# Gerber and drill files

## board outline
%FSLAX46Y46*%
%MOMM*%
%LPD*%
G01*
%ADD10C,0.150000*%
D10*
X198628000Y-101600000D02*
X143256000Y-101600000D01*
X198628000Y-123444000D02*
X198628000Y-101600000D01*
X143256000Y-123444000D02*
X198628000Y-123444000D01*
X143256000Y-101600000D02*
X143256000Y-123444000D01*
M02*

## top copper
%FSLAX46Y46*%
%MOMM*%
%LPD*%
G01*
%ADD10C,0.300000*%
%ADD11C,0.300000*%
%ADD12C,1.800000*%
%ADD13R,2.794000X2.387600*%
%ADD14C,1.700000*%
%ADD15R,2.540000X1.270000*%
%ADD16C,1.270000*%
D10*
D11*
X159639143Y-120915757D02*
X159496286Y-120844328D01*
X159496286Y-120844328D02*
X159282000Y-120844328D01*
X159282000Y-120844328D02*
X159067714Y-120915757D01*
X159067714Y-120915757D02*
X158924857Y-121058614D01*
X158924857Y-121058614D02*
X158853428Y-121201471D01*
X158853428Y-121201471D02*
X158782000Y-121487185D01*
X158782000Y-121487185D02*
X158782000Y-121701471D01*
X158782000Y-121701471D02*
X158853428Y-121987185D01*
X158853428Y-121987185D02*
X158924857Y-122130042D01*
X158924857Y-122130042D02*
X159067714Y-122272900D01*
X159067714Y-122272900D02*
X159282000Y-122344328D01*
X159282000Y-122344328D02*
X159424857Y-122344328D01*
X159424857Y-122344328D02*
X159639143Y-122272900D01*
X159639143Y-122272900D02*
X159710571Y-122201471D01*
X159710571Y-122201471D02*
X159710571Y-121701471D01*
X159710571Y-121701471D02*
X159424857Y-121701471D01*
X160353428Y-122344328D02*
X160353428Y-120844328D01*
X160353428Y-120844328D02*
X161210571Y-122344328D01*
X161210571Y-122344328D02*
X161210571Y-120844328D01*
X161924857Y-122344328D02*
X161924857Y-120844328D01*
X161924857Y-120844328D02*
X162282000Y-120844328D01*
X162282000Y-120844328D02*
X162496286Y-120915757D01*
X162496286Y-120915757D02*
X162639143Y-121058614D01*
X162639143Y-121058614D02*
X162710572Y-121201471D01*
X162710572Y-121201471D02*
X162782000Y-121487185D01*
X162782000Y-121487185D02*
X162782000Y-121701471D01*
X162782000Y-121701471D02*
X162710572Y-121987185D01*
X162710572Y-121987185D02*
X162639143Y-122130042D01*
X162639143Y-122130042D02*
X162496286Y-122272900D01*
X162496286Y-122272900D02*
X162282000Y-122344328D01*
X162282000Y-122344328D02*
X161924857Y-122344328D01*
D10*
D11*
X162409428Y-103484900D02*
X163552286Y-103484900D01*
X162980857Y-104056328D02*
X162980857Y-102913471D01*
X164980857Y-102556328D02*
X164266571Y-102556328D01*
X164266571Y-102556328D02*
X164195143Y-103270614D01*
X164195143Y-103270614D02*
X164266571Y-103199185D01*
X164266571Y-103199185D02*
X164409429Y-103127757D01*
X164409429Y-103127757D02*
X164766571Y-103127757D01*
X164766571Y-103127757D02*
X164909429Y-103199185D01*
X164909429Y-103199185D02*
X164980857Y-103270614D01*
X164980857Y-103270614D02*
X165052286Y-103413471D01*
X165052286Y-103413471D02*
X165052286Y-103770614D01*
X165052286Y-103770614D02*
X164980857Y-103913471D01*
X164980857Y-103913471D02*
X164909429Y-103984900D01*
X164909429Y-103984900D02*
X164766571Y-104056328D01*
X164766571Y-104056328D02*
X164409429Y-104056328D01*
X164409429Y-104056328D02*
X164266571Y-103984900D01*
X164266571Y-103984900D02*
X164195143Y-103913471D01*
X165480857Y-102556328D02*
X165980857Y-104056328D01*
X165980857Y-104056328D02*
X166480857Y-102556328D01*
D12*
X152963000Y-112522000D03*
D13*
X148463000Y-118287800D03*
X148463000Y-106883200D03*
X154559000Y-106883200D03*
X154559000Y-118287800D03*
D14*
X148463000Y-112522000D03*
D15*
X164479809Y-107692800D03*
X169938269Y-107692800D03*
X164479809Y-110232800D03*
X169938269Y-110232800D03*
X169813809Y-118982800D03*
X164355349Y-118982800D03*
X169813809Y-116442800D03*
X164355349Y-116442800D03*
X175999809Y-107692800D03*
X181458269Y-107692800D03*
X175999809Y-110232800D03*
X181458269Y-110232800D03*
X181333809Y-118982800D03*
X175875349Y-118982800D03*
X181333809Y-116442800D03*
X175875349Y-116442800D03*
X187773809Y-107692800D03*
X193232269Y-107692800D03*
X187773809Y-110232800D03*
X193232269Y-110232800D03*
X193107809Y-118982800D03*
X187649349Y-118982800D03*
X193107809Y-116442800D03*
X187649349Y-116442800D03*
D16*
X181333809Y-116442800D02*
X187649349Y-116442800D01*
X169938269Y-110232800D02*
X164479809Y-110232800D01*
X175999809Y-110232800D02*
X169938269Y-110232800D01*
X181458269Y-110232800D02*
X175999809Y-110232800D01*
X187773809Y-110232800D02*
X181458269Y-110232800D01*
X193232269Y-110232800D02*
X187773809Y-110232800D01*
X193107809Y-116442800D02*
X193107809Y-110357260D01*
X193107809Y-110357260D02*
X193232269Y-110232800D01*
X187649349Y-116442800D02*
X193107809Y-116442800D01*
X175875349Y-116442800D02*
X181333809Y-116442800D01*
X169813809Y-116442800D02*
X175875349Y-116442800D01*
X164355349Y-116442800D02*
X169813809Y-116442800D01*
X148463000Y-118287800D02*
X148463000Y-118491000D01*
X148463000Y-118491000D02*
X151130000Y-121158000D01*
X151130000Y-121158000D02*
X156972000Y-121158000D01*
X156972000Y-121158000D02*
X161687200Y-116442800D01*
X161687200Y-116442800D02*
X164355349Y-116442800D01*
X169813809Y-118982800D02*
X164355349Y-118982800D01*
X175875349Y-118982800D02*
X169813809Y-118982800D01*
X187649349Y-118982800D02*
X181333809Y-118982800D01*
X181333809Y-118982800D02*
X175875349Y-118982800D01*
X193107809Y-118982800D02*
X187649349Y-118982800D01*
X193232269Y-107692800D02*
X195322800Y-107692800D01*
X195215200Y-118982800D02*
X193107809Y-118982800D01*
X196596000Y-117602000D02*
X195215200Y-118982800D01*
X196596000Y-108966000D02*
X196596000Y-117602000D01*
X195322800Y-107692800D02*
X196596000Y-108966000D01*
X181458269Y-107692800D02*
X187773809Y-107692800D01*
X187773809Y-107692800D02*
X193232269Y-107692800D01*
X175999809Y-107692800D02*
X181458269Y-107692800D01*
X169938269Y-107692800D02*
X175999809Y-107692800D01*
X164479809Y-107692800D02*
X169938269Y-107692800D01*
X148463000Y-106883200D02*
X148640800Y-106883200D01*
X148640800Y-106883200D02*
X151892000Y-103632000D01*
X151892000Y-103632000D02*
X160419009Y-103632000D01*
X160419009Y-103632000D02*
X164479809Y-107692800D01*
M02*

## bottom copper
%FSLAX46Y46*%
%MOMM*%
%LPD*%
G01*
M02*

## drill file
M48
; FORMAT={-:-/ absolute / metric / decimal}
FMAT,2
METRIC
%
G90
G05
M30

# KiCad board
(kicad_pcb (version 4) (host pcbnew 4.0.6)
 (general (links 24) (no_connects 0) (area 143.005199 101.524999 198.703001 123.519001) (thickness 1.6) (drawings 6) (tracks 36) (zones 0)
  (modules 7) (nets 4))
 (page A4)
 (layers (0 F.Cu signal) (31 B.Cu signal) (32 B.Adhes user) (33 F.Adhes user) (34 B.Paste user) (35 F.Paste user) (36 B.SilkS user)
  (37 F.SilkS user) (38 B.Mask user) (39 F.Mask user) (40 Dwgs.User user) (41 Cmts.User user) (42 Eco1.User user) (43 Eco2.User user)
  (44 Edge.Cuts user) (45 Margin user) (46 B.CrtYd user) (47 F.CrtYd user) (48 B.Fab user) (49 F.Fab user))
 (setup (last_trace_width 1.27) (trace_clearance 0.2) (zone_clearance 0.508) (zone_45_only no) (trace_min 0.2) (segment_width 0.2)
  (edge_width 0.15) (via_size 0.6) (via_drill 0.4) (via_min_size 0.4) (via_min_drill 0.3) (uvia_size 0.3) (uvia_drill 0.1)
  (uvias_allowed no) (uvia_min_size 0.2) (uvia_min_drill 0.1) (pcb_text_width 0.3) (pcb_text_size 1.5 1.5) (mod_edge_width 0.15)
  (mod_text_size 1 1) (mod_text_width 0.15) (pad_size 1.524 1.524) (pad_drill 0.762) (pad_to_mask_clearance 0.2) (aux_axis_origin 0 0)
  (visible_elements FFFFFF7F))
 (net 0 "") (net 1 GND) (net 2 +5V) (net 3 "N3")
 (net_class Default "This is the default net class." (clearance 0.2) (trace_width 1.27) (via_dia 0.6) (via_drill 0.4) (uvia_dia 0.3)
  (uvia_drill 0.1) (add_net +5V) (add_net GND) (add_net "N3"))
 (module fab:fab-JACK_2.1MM (layer F.Cu) (at 150.876 112.522 270)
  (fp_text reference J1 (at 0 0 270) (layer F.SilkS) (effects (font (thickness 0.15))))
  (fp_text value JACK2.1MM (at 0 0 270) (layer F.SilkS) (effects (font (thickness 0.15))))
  (pad A smd circle (at 0 -2.087 270) (size 1.8 1.8) (layers F.Cu F.Paste F.Mask))
  (pad CONT smd rect (at 5.7658 2.413 270) (size 2.3876 2.794) (layers F.Cu F.Paste F.Mask) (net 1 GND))
  (pad PIN smd rect (at -5.6388 2.413 270) (size 2.3876 2.794) (layers F.Cu F.Paste F.Mask) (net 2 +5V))
  (pad PIN1 smd rect (at -5.6388 -3.683 270) (size 2.3876 2.794) (layers F.Cu F.Paste F.Mask))
  (pad SHUN smd rect (at 5.7658 -3.683 270) (size 2.3876 2.794) (layers F.Cu F.Paste F.Mask) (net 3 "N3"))
  (pad A smd circle (at 0 2.413 270) (size 1.7 1.7) (layers F.Cu F.Paste F.Mask)))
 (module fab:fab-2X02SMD (layer F.Cu) (at 167.019809 108.9628)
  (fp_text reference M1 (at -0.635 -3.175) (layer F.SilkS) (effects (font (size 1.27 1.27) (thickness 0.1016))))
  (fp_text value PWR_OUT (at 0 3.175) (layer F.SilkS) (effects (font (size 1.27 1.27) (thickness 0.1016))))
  (pad 1 smd rect (at -2.54 -1.27) (size 2.54 1.27) (layers F.Cu F.Paste F.Mask) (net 2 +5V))
  (pad 2 smd rect (at 2.91846 -1.27) (size 2.54 1.27) (layers F.Cu F.Paste F.Mask) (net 2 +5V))
  (pad 3 smd rect (at -2.54 1.27) (size 2.54 1.27) (layers F.Cu F.Paste F.Mask) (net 1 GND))
  (pad 4 smd rect (at 2.91846 1.27) (size 2.54 1.27) (layers F.Cu F.Paste F.Mask) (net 1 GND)))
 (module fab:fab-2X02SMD (layer F.Cu) (at 167.273809 117.7128 180)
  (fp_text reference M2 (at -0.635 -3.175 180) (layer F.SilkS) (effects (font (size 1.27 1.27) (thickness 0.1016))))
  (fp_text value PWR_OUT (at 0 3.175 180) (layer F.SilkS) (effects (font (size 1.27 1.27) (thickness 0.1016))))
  (pad 1 smd rect (at -2.54 -1.27 180) (size 2.54 1.27) (layers F.Cu F.Paste F.Mask) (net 2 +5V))
  (pad 2 smd rect (at 2.91846 -1.27 180) (size 2.54 1.27) (layers F.Cu F.Paste F.Mask) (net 2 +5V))
  (pad 3 smd rect (at -2.54 1.27 180) (size 2.54 1.27) (layers F.Cu F.Paste F.Mask) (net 1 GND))
  (pad 4 smd rect (at 2.91846 1.27 180) (size 2.54 1.27) (layers F.Cu F.Paste F.Mask) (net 1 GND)))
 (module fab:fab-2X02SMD (layer F.Cu) (at 178.539809 108.9628)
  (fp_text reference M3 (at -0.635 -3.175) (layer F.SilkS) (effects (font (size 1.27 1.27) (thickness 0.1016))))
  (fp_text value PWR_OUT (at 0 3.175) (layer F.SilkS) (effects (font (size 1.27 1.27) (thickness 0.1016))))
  (pad 1 smd rect (at -2.54 -1.27) (size 2.54 1.27) (layers F.Cu F.Paste F.Mask) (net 2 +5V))
  (pad 2 smd rect (at 2.91846 -1.27) (size 2.54 1.27) (layers F.Cu F.Paste F.Mask) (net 2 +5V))
  (pad 3 smd rect (at -2.54 1.27) (size 2.54 1.27) (layers F.Cu F.Paste F.Mask) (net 1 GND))
  (pad 4 smd rect (at 2.91846 1.27) (size 2.54 1.27) (layers F.Cu F.Paste F.Mask) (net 1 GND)))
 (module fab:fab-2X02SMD (layer F.Cu) (at 178.793809 117.7128 180)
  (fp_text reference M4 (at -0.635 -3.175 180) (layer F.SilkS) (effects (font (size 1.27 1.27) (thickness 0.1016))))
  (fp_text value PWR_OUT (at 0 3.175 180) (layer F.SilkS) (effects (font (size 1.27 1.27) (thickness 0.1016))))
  (pad 1 smd rect (at -2.54 -1.27 180) (size 2.54 1.27) (layers F.Cu F.Paste F.Mask) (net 2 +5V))
  (pad 2 smd rect (at 2.91846 -1.27 180) (size 2.54 1.27) (layers F.Cu F.Paste F.Mask) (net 2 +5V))
  (pad 3 smd rect (at -2.54 1.27 180) (size 2.54 1.27) (layers F.Cu F.Paste F.Mask) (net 1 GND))
  (pad 4 smd rect (at 2.91846 1.27 180) (size 2.54 1.27) (layers F.Cu F.Paste F.Mask) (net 1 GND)))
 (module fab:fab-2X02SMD (layer F.Cu) (at 190.313809 108.9628)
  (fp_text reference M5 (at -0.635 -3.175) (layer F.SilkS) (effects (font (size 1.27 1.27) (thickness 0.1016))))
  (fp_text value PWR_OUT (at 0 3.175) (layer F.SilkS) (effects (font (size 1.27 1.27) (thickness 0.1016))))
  (pad 1 smd rect (at -2.54 -1.27) (size 2.54 1.27) (layers F.Cu F.Paste F.Mask) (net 2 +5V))
  (pad 2 smd rect (at 2.91846 -1.27) (size 2.54 1.27) (layers F.Cu F.Paste F.Mask) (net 2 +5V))
  (pad 3 smd rect (at -2.54 1.27) (size 2.54 1.27) (layers F.Cu F.Paste F.Mask) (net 1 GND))
  (pad 4 smd rect (at 2.91846 1.27) (size 2.54 1.27) (layers F.Cu F.Paste F.Mask) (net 1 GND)))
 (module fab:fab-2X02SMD (layer F.Cu) (at 190.567809 117.7128 180)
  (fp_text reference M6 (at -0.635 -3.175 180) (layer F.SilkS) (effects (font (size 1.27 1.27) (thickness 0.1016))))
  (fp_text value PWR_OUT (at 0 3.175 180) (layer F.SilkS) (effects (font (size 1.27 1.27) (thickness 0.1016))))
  (pad 1 smd rect (at -2.54 -1.27 180) (size 2.54 1.27) (layers F.Cu F.Paste F.Mask) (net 2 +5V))
  (pad 2 smd rect (at 2.91846 -1.27 180) (size 2.54 1.27) (layers F.Cu F.Paste F.Mask) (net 2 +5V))
  (pad 3 smd rect (at -2.54 1.27 180) (size 2.54 1.27) (layers F.Cu F.Paste F.Mask) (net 1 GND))
  (pad 4 smd rect (at 2.91846 1.27 180) (size 2.54 1.27) (layers F.Cu F.Paste F.Mask) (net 1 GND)))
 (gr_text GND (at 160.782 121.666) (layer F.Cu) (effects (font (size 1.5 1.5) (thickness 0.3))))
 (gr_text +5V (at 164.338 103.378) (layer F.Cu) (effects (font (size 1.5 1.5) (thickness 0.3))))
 (gr_line (start 198.628 101.6) (end 143.256 101.6) (angle 90) (layer Edge.Cuts) (width 0.15))
 (gr_line (start 198.628 123.444) (end 198.628 101.6) (angle 90) (layer Edge.Cuts) (width 0.15))
 (gr_line (start 143.256 123.444) (end 198.628 123.444) (angle 90) (layer Edge.Cuts) (width 0.15))
 (gr_line (start 143.256 101.6) (end 143.256 123.444) (angle 90) (layer Edge.Cuts) (width 0.15))
 (segment (start 181.333809 116.4428) (end 187.649349 116.4428) (width 1.27) (layer F.Cu) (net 1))
 (segment (start 169.938269 110.2328) (end 164.479809 110.2328) (width 1.27) (layer F.Cu) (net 1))
 (segment (start 175.999809 110.2328) (end 169.938269 110.2328) (width 1.27) (layer F.Cu) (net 1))
 (segment (start 181.458269 110.2328) (end 175.999809 110.2328) (width 1.27) (layer F.Cu) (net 1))
 (segment (start 187.773809 110.2328) (end 181.458269 110.2328) (width 1.27) (layer F.Cu) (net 1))
 (segment (start 193.232269 110.2328) (end 187.773809 110.2328) (width 1.27) (layer F.Cu) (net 1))
 (segment (start 193.107809 116.4428) (end 193.107809 110.35726) (width 1.27) (layer F.Cu) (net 1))
 (segment (start 193.107809 110.35726) (end 193.232269 110.2328) (width 1.27) (layer F.Cu) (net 1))
 (segment (start 187.649349 116.4428) (end 193.107809 116.4428) (width 1.27) (layer F.Cu) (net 1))
 (segment (start 175.875349 116.4428) (end 181.333809 116.4428) (width 1.27) (layer F.Cu) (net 1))
 (segment (start 169.813809 116.4428) (end 175.875349 116.4428) (width 1.27) (layer F.Cu) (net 1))
 (segment (start 164.355349 116.4428) (end 169.813809 116.4428) (width 1.27) (layer F.Cu) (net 1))
 (segment (start 148.463 118.2878) (end 148.463 118.491) (width 1.27) (layer F.Cu) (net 1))
 (segment (start 148.463 118.491) (end 151.13 121.158) (width 1.27) (layer F.Cu) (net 1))
 (segment (start 151.13 121.158) (end 156.972 121.158) (width 1.27) (layer F.Cu) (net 1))
 (segment (start 156.972 121.158) (end 161.6872 116.4428) (width 1.27) (layer F.Cu) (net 1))
 (segment (start 161.6872 116.4428) (end 164.355349 116.4428) (width 1.27) (layer F.Cu) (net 1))
 (segment (start 169.813809 118.9828) (end 164.355349 118.9828) (width 1.27) (layer F.Cu) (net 2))
 (segment (start 175.875349 118.9828) (end 169.813809 118.9828) (width 1.27) (layer F.Cu) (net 2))
 (segment (start 187.649349 118.9828) (end 181.333809 118.9828) (width 1.27) (layer F.Cu) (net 2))
 (segment (start 181.333809 118.9828) (end 175.875349 118.9828) (width 1.27) (layer F.Cu) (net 2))
 (segment (start 193.107809 118.9828) (end 187.649349 118.9828) (width 1.27) (layer F.Cu) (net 2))
 (segment (start 193.232269 107.6928) (end 195.3228 107.6928) (width 1.27) (layer F.Cu) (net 2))
 (segment (start 195.2152 118.9828) (end 193.107809 118.9828) (width 1.27) (layer F.Cu) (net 2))
 (segment (start 196.596 117.602) (end 195.2152 118.9828) (width 1.27) (layer F.Cu) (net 2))
 (segment (start 196.596 108.966) (end 196.596 117.602) (width 1.27) (layer F.Cu) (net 2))
 (segment (start 195.3228 107.6928) (end 196.596 108.966) (width 1.27) (layer F.Cu) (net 2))
 (segment (start 181.458269 107.6928) (end 187.773809 107.6928) (width 1.27) (layer F.Cu) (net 2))
 (segment (start 187.773809 107.6928) (end 193.232269 107.6928) (width 1.27) (layer F.Cu) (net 2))
 (segment (start 175.999809 107.6928) (end 181.458269 107.6928) (width 1.27) (layer F.Cu) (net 2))
 (segment (start 169.938269 107.6928) (end 175.999809 107.6928) (width 1.27) (layer F.Cu) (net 2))
 (segment (start 164.479809 107.6928) (end 169.938269 107.6928) (width 1.27) (layer F.Cu) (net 2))
 (segment (start 148.463 106.8832) (end 148.6408 106.8832) (width 1.27) (layer F.Cu) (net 2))
 (segment (start 148.6408 106.8832) (end 151.892 103.632) (width 1.27) (layer F.Cu) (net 2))
 (segment (start 151.892 103.632) (end 160.419009 103.632) (width 1.27) (layer F.Cu) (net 2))
 (segment (start 160.419009 103.632) (end 164.479809 107.6928) (width 1.27) (layer F.Cu) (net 2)))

